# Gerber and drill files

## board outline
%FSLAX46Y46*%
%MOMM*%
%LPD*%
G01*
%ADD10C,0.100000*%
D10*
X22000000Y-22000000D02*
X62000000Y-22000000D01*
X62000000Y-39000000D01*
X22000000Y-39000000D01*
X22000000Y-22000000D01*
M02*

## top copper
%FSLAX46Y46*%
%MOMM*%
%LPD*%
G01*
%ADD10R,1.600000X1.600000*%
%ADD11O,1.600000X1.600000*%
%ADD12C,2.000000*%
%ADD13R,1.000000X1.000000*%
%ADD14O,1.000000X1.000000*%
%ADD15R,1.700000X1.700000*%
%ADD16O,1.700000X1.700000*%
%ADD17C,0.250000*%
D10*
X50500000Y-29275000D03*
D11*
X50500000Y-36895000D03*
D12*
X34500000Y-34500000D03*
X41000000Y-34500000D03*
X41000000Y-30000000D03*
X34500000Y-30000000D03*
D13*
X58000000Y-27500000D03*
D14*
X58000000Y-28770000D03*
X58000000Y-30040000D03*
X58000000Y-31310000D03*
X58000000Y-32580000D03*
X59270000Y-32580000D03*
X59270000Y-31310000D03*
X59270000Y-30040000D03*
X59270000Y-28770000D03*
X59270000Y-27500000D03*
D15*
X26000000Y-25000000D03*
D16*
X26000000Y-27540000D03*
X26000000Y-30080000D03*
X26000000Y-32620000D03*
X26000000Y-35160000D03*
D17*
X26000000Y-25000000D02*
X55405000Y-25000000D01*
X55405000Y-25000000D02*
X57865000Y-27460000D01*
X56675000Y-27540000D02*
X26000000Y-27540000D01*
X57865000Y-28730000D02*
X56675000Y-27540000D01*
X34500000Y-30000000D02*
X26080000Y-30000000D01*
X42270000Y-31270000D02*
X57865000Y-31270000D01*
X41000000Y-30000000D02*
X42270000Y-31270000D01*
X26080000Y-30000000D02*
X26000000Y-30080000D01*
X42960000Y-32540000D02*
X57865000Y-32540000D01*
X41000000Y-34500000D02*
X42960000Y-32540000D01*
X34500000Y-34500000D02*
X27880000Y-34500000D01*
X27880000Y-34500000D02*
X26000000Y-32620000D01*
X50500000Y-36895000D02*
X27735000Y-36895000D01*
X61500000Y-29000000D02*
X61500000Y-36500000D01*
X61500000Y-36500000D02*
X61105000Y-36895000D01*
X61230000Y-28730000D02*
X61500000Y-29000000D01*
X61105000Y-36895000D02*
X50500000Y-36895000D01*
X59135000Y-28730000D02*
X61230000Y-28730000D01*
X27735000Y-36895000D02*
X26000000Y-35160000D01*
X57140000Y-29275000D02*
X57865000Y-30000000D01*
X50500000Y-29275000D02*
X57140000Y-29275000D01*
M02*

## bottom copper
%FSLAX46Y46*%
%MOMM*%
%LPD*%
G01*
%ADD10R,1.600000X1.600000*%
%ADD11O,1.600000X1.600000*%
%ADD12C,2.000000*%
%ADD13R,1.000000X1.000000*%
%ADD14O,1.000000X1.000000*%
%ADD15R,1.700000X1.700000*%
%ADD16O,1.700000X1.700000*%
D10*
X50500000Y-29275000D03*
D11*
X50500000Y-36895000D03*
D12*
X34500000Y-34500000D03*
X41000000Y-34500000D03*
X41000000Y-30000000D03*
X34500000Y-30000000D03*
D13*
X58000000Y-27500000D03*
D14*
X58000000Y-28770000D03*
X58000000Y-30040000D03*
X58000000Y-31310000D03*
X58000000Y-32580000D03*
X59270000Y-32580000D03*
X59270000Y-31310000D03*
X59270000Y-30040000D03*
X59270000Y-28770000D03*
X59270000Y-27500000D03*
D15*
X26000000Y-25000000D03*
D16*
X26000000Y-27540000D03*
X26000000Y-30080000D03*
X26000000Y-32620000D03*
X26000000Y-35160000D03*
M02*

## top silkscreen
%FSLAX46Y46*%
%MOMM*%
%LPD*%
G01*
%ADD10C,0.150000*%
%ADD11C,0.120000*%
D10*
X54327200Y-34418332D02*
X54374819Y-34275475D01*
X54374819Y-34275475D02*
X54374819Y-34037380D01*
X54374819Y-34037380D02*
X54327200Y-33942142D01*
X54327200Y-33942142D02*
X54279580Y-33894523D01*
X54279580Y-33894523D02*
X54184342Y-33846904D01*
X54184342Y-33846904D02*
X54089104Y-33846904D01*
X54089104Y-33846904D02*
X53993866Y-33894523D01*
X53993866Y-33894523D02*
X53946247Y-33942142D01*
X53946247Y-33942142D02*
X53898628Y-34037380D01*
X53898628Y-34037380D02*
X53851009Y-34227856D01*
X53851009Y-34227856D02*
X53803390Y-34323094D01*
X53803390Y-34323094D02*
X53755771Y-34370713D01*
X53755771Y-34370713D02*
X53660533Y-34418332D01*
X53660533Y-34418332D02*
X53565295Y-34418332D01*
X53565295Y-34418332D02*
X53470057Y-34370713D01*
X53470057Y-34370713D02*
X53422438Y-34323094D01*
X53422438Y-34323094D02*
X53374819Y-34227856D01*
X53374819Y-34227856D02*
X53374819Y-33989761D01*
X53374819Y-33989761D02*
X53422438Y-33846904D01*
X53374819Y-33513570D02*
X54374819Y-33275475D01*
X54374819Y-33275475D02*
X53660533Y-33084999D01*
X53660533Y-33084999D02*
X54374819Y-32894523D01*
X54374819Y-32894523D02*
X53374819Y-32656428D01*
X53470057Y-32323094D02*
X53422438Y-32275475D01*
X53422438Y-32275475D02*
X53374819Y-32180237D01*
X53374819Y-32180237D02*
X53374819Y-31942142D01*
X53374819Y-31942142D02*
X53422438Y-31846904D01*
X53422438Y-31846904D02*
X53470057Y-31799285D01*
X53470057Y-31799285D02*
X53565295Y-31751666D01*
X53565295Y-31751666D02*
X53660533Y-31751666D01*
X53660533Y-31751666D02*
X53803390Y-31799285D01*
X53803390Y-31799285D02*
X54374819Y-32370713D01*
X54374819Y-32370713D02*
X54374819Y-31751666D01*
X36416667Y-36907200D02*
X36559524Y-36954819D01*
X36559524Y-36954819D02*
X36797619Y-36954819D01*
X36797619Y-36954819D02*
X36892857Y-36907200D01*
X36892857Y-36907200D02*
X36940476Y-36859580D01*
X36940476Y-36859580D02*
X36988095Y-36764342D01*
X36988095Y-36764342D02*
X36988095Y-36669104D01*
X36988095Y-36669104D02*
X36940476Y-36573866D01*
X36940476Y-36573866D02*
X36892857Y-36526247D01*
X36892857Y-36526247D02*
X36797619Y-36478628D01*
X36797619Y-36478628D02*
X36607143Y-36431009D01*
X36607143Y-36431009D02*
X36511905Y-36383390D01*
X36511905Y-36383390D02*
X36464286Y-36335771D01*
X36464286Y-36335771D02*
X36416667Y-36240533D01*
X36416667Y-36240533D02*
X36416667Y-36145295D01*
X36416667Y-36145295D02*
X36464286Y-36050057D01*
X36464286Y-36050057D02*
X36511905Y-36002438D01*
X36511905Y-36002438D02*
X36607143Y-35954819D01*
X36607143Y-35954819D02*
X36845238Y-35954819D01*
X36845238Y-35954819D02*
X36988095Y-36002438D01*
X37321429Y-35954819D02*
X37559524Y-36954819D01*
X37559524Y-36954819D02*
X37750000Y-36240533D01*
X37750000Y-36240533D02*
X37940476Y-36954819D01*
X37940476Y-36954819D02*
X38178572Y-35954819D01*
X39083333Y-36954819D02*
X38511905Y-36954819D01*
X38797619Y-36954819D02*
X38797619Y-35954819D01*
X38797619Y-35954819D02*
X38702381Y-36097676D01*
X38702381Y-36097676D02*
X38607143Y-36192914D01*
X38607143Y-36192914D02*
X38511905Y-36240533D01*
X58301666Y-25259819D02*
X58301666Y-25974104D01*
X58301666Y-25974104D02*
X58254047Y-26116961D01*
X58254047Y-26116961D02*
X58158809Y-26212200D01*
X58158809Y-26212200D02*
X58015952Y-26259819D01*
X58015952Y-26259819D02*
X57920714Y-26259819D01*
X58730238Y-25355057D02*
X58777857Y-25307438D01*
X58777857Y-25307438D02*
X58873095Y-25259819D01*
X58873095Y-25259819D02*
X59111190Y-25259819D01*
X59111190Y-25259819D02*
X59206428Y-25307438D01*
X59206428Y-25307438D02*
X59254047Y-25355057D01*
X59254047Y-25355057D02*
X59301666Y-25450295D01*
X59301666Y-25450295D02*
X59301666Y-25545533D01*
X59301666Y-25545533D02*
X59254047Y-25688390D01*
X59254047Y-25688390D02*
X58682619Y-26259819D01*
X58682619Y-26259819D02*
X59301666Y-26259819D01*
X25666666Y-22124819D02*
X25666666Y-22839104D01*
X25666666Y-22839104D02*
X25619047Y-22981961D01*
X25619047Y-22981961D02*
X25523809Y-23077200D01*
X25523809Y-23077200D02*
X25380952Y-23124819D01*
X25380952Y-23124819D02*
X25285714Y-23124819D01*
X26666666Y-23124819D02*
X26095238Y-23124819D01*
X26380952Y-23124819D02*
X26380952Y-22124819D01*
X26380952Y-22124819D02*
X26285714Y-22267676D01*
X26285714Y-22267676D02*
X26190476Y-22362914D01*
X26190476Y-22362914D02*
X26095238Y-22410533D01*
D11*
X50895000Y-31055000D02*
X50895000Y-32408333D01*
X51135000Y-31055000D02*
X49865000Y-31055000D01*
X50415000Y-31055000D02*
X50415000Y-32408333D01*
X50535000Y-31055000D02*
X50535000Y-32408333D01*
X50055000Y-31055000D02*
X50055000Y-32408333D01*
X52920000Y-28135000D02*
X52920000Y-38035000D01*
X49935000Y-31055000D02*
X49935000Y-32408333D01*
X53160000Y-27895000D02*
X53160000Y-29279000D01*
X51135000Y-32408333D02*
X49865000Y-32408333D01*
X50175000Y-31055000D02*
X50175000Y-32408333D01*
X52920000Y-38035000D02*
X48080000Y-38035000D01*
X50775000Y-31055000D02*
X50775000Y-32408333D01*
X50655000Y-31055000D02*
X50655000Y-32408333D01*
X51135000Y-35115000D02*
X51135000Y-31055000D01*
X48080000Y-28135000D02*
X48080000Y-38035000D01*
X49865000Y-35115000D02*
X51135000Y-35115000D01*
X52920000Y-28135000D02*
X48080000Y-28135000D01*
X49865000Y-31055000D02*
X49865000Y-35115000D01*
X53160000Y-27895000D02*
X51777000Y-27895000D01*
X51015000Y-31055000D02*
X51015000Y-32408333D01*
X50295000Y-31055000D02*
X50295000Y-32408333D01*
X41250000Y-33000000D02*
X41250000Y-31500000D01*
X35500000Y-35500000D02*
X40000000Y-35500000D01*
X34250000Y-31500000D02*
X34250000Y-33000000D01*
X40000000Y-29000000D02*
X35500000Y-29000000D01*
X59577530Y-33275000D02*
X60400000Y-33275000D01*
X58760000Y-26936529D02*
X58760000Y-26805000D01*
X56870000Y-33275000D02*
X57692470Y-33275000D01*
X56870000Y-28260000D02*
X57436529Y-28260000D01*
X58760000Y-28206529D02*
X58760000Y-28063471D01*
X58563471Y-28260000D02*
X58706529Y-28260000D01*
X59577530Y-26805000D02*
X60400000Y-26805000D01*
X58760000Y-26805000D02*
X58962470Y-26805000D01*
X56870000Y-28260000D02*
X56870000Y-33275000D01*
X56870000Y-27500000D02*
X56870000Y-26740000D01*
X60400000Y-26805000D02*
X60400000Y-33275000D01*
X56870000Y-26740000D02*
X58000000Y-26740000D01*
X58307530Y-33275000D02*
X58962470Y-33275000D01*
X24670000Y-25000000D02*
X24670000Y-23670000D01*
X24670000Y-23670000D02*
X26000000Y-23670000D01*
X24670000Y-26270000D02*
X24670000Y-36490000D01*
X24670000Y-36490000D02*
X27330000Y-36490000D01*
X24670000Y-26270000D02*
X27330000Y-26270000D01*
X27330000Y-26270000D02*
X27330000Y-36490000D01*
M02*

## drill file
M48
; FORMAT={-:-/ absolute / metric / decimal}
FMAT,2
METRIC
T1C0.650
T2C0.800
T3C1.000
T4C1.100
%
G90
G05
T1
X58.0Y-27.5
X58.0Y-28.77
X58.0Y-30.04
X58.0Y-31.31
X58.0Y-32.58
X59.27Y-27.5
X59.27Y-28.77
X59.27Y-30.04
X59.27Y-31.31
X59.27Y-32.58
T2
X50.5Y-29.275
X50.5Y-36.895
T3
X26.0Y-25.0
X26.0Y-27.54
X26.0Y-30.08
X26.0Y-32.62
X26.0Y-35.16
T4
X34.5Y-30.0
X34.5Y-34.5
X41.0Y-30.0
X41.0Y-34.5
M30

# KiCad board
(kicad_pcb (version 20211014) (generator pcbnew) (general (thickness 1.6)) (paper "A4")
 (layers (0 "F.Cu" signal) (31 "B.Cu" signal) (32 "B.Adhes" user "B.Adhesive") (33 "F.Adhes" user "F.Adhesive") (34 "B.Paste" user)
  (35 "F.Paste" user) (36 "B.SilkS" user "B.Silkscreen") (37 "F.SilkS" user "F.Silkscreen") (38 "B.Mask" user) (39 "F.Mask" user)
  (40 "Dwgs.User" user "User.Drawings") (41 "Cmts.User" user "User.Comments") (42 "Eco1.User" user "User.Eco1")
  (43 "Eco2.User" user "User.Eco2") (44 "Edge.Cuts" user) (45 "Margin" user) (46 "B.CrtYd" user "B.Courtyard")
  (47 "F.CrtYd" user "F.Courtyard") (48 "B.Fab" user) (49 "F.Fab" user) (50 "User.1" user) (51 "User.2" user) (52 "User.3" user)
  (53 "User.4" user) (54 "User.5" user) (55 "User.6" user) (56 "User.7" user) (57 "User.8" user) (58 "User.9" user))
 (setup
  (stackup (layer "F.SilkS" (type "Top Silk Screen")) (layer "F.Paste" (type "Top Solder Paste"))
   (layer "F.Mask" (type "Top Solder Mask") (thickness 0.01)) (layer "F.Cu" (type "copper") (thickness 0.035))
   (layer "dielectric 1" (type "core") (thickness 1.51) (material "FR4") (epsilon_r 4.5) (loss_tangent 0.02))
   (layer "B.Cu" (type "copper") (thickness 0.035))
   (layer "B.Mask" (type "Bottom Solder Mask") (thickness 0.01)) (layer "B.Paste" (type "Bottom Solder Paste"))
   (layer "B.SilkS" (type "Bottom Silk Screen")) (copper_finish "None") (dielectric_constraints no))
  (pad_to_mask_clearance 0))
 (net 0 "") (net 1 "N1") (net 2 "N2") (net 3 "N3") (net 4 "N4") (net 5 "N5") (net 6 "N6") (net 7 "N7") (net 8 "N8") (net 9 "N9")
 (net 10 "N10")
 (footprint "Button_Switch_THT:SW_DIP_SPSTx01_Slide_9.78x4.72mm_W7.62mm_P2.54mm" (layer "F.Cu") (at 50.5 29.275 -90)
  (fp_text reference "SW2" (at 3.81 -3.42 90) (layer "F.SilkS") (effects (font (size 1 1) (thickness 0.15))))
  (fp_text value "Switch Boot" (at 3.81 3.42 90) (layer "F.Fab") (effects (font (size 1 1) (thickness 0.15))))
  (fp_line (start 1.78 -0.395) (end 3.133333 -0.395) (layer "F.SilkS") (width 0.12))
  (fp_line (start 1.78 -0.635) (end 1.78 0.635) (layer "F.SilkS") (width 0.12))
  (fp_line (start 1.78 0.085) (end 3.133333 0.085) (layer "F.SilkS") (width 0.12))
  (fp_line (start 1.78 -0.035) (end 3.133333 -0.035) (layer "F.SilkS") (width 0.12))
  (fp_line (start 1.78 0.445) (end 3.133333 0.445) (layer "F.SilkS") (width 0.12))
  (fp_line (start -1.14 -2.42) (end 8.76 -2.42) (layer "F.SilkS") (width 0.12))
  (fp_line (start 1.78 0.565) (end 3.133333 0.565) (layer "F.SilkS") (width 0.12))
  (fp_line (start -1.38 -2.66) (end 0.004 -2.66) (layer "F.SilkS") (width 0.12))
  (fp_line (start 3.133333 -0.635) (end 3.133333 0.635) (layer "F.SilkS") (width 0.12))
  (fp_line (start 1.78 0.325) (end 3.133333 0.325) (layer "F.SilkS") (width 0.12))
  (fp_line (start 8.76 -2.42) (end 8.76 2.42) (layer "F.SilkS") (width 0.12))
  (fp_line (start 1.78 -0.275) (end 3.133333 -0.275) (layer "F.SilkS") (width 0.12))
  (fp_line (start 1.78 -0.155) (end 3.133333 -0.155) (layer "F.SilkS") (width 0.12))
  (fp_line (start 5.84 -0.635) (end 1.78 -0.635) (layer "F.SilkS") (width 0.12))
  (fp_line (start -1.14 2.42) (end 8.76 2.42) (layer "F.SilkS") (width 0.12))
  (fp_line (start 5.84 0.635) (end 5.84 -0.635) (layer "F.SilkS") (width 0.12))
  (fp_line (start -1.14 -2.42) (end -1.14 2.42) (layer "F.SilkS") (width 0.12))
  (fp_line (start 1.78 0.635) (end 5.84 0.635) (layer "F.SilkS") (width 0.12))
  (fp_line (start -1.38 -2.66) (end -1.38 -1.277) (layer "F.SilkS") (width 0.12))
  (fp_line (start 1.78 -0.515) (end 3.133333 -0.515) (layer "F.SilkS") (width 0.12))
  (fp_line (start 1.78 0.205) (end 3.133333 0.205) (layer "F.SilkS") (width 0.12))
  (pad "1" thru_hole rect (at 0 0 270) (size 1.6 1.6) (drill 0.8) (layers *.Cu *.Mask) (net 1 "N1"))
  (pad "2" thru_hole oval (at 7.62 0 270) (size 1.6 1.6) (drill 0.8) (layers *.Cu *.Mask) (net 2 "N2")))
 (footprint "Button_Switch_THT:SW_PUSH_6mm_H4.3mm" (layer "F.Cu") (at 41 34.5 180)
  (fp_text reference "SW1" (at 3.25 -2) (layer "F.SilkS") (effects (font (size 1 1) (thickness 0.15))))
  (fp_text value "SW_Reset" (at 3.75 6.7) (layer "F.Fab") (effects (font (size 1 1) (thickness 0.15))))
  (fp_line (start -0.25 1.5) (end -0.25 3) (layer "F.SilkS") (width 0.12))
  (fp_line (start 5.5 -1) (end 1 -1) (layer "F.SilkS") (width 0.12))
  (fp_line (start 6.75 3) (end 6.75 1.5) (layer "F.SilkS") (width 0.12))
  (fp_line (start 1 5.5) (end 5.5 5.5) (layer "F.SilkS") (width 0.12))
  (pad "1" thru_hole circle (at 6.5 0 270) (size 2 2) (drill 1.1) (layers *.Cu *.Mask) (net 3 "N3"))
  (pad "1" thru_hole circle (at 0 0 270) (size 2 2) (drill 1.1) (layers *.Cu *.Mask) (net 3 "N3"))
  (pad "2" thru_hole circle (at 0 4.5 270) (size 2 2) (drill 1.1) (layers *.Cu *.Mask) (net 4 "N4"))
  (pad "2" thru_hole circle (at 6.5 4.5 270) (size 2 2) (drill 1.1) (layers *.Cu *.Mask) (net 4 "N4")))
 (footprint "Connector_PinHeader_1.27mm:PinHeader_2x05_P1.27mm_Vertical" (layer "F.Cu") (at 58 27.5)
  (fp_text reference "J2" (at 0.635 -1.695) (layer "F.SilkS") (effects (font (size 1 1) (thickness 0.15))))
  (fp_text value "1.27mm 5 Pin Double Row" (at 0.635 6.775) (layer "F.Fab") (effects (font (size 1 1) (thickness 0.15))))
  (fp_line (start 1.57753 5.775) (end 2.4 5.775) (layer "F.SilkS") (width 0.12))
  (fp_line (start 0.76 -0.563471) (end 0.76 -0.695) (layer "F.SilkS") (width 0.12))
  (fp_line (start -1.13 5.775) (end -0.30753 5.775) (layer "F.SilkS") (width 0.12))
  (fp_line (start -1.13 0.76) (end -0.563471 0.76) (layer "F.SilkS") (width 0.12))
  (fp_line (start 0.76 0.706529) (end 0.76 0.563471) (layer "F.SilkS") (width 0.12))
  (fp_line (start 0.563471 0.76) (end 0.706529 0.76) (layer "F.SilkS") (width 0.12))
  (fp_line (start 1.57753 -0.695) (end 2.4 -0.695) (layer "F.SilkS") (width 0.12))
  (fp_line (start 0.76 -0.695) (end 0.96247 -0.695) (layer "F.SilkS") (width 0.12))
  (fp_line (start -1.13 0.76) (end -1.13 5.775) (layer "F.SilkS") (width 0.12))
  (fp_line (start -1.13 0) (end -1.13 -0.76) (layer "F.SilkS") (width 0.12))
  (fp_line (start 2.4 -0.695) (end 2.4 5.775) (layer "F.SilkS") (width 0.12))
  (fp_line (start -1.13 -0.76) (end 0 -0.76) (layer "F.SilkS") (width 0.12))
  (fp_line (start 0.30753 5.775) (end 0.96247 5.775) (layer "F.SilkS") (width 0.12))
  (pad "1" thru_hole rect (at 0 0) (size 1 1) (drill 0.65) (layers *.Cu *.Mask) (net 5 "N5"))
  (pad "2" thru_hole oval (at 0 1.27) (size 1 1) (drill 0.65) (layers *.Cu *.Mask) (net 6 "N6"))
  (pad "3" thru_hole oval (at 0 2.54) (size 1 1) (drill 0.65) (layers *.Cu *.Mask) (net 1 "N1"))
  (pad "4" thru_hole oval (at 0 3.81) (size 1 1) (drill 0.65) (layers *.Cu *.Mask) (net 4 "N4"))
  (pad "5" thru_hole oval (at 0 5.08) (size 1 1) (drill 0.65) (layers *.Cu *.Mask) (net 3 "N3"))
  (pad "6" thru_hole oval (at 1.27 5.08) (size 1 1) (drill 0.65) (layers *.Cu *.Mask) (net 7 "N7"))
  (pad "7" thru_hole oval (at 1.27 3.81) (size 1 1) (drill 0.65) (layers *.Cu *.Mask) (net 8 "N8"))
  (pad "8" thru_hole oval (at 1.27 2.54) (size 1 1) (drill 0.65) (layers *.Cu *.Mask) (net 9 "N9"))
  (pad "9" thru_hole oval (at 1.27 1.27) (size 1 1) (drill 0.65) (layers *.Cu *.Mask) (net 2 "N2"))
  (pad "10" thru_hole oval (at 1.27 0) (size 1 1) (drill 0.65) (layers *.Cu *.Mask) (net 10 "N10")))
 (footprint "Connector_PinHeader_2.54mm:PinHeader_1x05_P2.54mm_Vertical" (layer "F.Cu") (at 26 25)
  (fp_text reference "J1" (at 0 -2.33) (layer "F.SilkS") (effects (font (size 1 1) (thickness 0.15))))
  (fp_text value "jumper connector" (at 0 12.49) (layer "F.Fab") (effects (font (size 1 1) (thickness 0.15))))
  (fp_line (start -1.33 0) (end -1.33 -1.33) (layer "F.SilkS") (width 0.12))
  (fp_line (start -1.33 -1.33) (end 0 -1.33) (layer "F.SilkS") (width 0.12))
  (fp_line (start -1.33 1.27) (end -1.33 11.49) (layer "F.SilkS") (width 0.12))
  (fp_line (start -1.33 11.49) (end 1.33 11.49) (layer "F.SilkS") (width 0.12))
  (fp_line (start -1.33 1.27) (end 1.33 1.27) (layer "F.SilkS") (width 0.12))
  (fp_line (start 1.33 1.27) (end 1.33 11.49) (layer "F.SilkS") (width 0.12))
  (pad "1" thru_hole rect (at 0 0) (size 1.7 1.7) (drill 1) (layers *.Cu *.Mask) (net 5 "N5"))
  (pad "2" thru_hole oval (at 0 2.54) (size 1.7 1.7) (drill 1) (layers *.Cu *.Mask) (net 6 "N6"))
  (pad "3" thru_hole oval (at 0 5.08) (size 1.7 1.7) (drill 1) (layers *.Cu *.Mask) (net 4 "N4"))
  (pad "4" thru_hole oval (at 0 7.62) (size 1.7 1.7) (drill 1) (layers *.Cu *.Mask) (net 3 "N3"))
  (pad "5" thru_hole oval (at 0 10.16) (size 1.7 1.7) (drill 1) (layers *.Cu *.Mask) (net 2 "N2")))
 (gr_rect (start 62 22) (end 22 39) (layer "Edge.Cuts") (width 0.1) (fill none))
 (segment (start 26 25) (end 55.405 25) (width 0.25) (layer "F.Cu") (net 5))
 (segment (start 55.405 25) (end 57.865 27.46) (width 0.25) (layer "F.Cu") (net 5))
 (segment (start 56.675 27.54) (end 26 27.54) (width 0.25) (layer "F.Cu") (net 6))
 (segment (start 57.865 28.73) (end 56.675 27.54) (width 0.25) (layer "F.Cu") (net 6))
 (segment (start 34.5 30) (end 26.08 30) (width 0.25) (layer "F.Cu") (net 4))
 (segment (start 42.27 31.27) (end 57.865 31.27) (width 0.25) (layer "F.Cu") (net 4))
 (segment (start 41 30) (end 42.27 31.27) (width 0.25) (layer "F.Cu") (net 4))
 (segment (start 26.08 30) (end 26 30.08) (width 0.25) (layer "F.Cu") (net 4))
 (segment (start 42.96 32.54) (end 57.865 32.54) (width 0.25) (layer "F.Cu") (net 3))
 (segment (start 41 34.5) (end 42.96 32.54) (width 0.25) (layer "F.Cu") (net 3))
 (segment (start 34.5 34.5) (end 27.88 34.5) (width 0.25) (layer "F.Cu") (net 3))
 (segment (start 27.88 34.5) (end 26 32.62) (width 0.25) (layer "F.Cu") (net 3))
 (segment (start 50.5 36.895) (end 27.735 36.895) (width 0.25) (layer "F.Cu") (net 2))
 (segment (start 61.5 29) (end 61.5 36.5) (width 0.25) (layer "F.Cu") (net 2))
 (segment (start 61.5 36.5) (end 61.105 36.895) (width 0.25) (layer "F.Cu") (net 2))
 (segment (start 61.23 28.73) (end 61.5 29) (width 0.25) (layer "F.Cu") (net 2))
 (segment (start 61.105 36.895) (end 50.5 36.895) (width 0.25) (layer "F.Cu") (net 2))
 (segment (start 59.135 28.73) (end 61.23 28.73) (width 0.25) (layer "F.Cu") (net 2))
 (segment (start 27.735 36.895) (end 26 35.16) (width 0.25) (layer "F.Cu") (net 2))
 (segment (start 57.14 29.275) (end 57.865 30) (width 0.25) (layer "F.Cu") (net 1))
 (segment (start 50.5 29.275) (end 57.14 29.275) (width 0.25) (layer "F.Cu") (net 1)))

